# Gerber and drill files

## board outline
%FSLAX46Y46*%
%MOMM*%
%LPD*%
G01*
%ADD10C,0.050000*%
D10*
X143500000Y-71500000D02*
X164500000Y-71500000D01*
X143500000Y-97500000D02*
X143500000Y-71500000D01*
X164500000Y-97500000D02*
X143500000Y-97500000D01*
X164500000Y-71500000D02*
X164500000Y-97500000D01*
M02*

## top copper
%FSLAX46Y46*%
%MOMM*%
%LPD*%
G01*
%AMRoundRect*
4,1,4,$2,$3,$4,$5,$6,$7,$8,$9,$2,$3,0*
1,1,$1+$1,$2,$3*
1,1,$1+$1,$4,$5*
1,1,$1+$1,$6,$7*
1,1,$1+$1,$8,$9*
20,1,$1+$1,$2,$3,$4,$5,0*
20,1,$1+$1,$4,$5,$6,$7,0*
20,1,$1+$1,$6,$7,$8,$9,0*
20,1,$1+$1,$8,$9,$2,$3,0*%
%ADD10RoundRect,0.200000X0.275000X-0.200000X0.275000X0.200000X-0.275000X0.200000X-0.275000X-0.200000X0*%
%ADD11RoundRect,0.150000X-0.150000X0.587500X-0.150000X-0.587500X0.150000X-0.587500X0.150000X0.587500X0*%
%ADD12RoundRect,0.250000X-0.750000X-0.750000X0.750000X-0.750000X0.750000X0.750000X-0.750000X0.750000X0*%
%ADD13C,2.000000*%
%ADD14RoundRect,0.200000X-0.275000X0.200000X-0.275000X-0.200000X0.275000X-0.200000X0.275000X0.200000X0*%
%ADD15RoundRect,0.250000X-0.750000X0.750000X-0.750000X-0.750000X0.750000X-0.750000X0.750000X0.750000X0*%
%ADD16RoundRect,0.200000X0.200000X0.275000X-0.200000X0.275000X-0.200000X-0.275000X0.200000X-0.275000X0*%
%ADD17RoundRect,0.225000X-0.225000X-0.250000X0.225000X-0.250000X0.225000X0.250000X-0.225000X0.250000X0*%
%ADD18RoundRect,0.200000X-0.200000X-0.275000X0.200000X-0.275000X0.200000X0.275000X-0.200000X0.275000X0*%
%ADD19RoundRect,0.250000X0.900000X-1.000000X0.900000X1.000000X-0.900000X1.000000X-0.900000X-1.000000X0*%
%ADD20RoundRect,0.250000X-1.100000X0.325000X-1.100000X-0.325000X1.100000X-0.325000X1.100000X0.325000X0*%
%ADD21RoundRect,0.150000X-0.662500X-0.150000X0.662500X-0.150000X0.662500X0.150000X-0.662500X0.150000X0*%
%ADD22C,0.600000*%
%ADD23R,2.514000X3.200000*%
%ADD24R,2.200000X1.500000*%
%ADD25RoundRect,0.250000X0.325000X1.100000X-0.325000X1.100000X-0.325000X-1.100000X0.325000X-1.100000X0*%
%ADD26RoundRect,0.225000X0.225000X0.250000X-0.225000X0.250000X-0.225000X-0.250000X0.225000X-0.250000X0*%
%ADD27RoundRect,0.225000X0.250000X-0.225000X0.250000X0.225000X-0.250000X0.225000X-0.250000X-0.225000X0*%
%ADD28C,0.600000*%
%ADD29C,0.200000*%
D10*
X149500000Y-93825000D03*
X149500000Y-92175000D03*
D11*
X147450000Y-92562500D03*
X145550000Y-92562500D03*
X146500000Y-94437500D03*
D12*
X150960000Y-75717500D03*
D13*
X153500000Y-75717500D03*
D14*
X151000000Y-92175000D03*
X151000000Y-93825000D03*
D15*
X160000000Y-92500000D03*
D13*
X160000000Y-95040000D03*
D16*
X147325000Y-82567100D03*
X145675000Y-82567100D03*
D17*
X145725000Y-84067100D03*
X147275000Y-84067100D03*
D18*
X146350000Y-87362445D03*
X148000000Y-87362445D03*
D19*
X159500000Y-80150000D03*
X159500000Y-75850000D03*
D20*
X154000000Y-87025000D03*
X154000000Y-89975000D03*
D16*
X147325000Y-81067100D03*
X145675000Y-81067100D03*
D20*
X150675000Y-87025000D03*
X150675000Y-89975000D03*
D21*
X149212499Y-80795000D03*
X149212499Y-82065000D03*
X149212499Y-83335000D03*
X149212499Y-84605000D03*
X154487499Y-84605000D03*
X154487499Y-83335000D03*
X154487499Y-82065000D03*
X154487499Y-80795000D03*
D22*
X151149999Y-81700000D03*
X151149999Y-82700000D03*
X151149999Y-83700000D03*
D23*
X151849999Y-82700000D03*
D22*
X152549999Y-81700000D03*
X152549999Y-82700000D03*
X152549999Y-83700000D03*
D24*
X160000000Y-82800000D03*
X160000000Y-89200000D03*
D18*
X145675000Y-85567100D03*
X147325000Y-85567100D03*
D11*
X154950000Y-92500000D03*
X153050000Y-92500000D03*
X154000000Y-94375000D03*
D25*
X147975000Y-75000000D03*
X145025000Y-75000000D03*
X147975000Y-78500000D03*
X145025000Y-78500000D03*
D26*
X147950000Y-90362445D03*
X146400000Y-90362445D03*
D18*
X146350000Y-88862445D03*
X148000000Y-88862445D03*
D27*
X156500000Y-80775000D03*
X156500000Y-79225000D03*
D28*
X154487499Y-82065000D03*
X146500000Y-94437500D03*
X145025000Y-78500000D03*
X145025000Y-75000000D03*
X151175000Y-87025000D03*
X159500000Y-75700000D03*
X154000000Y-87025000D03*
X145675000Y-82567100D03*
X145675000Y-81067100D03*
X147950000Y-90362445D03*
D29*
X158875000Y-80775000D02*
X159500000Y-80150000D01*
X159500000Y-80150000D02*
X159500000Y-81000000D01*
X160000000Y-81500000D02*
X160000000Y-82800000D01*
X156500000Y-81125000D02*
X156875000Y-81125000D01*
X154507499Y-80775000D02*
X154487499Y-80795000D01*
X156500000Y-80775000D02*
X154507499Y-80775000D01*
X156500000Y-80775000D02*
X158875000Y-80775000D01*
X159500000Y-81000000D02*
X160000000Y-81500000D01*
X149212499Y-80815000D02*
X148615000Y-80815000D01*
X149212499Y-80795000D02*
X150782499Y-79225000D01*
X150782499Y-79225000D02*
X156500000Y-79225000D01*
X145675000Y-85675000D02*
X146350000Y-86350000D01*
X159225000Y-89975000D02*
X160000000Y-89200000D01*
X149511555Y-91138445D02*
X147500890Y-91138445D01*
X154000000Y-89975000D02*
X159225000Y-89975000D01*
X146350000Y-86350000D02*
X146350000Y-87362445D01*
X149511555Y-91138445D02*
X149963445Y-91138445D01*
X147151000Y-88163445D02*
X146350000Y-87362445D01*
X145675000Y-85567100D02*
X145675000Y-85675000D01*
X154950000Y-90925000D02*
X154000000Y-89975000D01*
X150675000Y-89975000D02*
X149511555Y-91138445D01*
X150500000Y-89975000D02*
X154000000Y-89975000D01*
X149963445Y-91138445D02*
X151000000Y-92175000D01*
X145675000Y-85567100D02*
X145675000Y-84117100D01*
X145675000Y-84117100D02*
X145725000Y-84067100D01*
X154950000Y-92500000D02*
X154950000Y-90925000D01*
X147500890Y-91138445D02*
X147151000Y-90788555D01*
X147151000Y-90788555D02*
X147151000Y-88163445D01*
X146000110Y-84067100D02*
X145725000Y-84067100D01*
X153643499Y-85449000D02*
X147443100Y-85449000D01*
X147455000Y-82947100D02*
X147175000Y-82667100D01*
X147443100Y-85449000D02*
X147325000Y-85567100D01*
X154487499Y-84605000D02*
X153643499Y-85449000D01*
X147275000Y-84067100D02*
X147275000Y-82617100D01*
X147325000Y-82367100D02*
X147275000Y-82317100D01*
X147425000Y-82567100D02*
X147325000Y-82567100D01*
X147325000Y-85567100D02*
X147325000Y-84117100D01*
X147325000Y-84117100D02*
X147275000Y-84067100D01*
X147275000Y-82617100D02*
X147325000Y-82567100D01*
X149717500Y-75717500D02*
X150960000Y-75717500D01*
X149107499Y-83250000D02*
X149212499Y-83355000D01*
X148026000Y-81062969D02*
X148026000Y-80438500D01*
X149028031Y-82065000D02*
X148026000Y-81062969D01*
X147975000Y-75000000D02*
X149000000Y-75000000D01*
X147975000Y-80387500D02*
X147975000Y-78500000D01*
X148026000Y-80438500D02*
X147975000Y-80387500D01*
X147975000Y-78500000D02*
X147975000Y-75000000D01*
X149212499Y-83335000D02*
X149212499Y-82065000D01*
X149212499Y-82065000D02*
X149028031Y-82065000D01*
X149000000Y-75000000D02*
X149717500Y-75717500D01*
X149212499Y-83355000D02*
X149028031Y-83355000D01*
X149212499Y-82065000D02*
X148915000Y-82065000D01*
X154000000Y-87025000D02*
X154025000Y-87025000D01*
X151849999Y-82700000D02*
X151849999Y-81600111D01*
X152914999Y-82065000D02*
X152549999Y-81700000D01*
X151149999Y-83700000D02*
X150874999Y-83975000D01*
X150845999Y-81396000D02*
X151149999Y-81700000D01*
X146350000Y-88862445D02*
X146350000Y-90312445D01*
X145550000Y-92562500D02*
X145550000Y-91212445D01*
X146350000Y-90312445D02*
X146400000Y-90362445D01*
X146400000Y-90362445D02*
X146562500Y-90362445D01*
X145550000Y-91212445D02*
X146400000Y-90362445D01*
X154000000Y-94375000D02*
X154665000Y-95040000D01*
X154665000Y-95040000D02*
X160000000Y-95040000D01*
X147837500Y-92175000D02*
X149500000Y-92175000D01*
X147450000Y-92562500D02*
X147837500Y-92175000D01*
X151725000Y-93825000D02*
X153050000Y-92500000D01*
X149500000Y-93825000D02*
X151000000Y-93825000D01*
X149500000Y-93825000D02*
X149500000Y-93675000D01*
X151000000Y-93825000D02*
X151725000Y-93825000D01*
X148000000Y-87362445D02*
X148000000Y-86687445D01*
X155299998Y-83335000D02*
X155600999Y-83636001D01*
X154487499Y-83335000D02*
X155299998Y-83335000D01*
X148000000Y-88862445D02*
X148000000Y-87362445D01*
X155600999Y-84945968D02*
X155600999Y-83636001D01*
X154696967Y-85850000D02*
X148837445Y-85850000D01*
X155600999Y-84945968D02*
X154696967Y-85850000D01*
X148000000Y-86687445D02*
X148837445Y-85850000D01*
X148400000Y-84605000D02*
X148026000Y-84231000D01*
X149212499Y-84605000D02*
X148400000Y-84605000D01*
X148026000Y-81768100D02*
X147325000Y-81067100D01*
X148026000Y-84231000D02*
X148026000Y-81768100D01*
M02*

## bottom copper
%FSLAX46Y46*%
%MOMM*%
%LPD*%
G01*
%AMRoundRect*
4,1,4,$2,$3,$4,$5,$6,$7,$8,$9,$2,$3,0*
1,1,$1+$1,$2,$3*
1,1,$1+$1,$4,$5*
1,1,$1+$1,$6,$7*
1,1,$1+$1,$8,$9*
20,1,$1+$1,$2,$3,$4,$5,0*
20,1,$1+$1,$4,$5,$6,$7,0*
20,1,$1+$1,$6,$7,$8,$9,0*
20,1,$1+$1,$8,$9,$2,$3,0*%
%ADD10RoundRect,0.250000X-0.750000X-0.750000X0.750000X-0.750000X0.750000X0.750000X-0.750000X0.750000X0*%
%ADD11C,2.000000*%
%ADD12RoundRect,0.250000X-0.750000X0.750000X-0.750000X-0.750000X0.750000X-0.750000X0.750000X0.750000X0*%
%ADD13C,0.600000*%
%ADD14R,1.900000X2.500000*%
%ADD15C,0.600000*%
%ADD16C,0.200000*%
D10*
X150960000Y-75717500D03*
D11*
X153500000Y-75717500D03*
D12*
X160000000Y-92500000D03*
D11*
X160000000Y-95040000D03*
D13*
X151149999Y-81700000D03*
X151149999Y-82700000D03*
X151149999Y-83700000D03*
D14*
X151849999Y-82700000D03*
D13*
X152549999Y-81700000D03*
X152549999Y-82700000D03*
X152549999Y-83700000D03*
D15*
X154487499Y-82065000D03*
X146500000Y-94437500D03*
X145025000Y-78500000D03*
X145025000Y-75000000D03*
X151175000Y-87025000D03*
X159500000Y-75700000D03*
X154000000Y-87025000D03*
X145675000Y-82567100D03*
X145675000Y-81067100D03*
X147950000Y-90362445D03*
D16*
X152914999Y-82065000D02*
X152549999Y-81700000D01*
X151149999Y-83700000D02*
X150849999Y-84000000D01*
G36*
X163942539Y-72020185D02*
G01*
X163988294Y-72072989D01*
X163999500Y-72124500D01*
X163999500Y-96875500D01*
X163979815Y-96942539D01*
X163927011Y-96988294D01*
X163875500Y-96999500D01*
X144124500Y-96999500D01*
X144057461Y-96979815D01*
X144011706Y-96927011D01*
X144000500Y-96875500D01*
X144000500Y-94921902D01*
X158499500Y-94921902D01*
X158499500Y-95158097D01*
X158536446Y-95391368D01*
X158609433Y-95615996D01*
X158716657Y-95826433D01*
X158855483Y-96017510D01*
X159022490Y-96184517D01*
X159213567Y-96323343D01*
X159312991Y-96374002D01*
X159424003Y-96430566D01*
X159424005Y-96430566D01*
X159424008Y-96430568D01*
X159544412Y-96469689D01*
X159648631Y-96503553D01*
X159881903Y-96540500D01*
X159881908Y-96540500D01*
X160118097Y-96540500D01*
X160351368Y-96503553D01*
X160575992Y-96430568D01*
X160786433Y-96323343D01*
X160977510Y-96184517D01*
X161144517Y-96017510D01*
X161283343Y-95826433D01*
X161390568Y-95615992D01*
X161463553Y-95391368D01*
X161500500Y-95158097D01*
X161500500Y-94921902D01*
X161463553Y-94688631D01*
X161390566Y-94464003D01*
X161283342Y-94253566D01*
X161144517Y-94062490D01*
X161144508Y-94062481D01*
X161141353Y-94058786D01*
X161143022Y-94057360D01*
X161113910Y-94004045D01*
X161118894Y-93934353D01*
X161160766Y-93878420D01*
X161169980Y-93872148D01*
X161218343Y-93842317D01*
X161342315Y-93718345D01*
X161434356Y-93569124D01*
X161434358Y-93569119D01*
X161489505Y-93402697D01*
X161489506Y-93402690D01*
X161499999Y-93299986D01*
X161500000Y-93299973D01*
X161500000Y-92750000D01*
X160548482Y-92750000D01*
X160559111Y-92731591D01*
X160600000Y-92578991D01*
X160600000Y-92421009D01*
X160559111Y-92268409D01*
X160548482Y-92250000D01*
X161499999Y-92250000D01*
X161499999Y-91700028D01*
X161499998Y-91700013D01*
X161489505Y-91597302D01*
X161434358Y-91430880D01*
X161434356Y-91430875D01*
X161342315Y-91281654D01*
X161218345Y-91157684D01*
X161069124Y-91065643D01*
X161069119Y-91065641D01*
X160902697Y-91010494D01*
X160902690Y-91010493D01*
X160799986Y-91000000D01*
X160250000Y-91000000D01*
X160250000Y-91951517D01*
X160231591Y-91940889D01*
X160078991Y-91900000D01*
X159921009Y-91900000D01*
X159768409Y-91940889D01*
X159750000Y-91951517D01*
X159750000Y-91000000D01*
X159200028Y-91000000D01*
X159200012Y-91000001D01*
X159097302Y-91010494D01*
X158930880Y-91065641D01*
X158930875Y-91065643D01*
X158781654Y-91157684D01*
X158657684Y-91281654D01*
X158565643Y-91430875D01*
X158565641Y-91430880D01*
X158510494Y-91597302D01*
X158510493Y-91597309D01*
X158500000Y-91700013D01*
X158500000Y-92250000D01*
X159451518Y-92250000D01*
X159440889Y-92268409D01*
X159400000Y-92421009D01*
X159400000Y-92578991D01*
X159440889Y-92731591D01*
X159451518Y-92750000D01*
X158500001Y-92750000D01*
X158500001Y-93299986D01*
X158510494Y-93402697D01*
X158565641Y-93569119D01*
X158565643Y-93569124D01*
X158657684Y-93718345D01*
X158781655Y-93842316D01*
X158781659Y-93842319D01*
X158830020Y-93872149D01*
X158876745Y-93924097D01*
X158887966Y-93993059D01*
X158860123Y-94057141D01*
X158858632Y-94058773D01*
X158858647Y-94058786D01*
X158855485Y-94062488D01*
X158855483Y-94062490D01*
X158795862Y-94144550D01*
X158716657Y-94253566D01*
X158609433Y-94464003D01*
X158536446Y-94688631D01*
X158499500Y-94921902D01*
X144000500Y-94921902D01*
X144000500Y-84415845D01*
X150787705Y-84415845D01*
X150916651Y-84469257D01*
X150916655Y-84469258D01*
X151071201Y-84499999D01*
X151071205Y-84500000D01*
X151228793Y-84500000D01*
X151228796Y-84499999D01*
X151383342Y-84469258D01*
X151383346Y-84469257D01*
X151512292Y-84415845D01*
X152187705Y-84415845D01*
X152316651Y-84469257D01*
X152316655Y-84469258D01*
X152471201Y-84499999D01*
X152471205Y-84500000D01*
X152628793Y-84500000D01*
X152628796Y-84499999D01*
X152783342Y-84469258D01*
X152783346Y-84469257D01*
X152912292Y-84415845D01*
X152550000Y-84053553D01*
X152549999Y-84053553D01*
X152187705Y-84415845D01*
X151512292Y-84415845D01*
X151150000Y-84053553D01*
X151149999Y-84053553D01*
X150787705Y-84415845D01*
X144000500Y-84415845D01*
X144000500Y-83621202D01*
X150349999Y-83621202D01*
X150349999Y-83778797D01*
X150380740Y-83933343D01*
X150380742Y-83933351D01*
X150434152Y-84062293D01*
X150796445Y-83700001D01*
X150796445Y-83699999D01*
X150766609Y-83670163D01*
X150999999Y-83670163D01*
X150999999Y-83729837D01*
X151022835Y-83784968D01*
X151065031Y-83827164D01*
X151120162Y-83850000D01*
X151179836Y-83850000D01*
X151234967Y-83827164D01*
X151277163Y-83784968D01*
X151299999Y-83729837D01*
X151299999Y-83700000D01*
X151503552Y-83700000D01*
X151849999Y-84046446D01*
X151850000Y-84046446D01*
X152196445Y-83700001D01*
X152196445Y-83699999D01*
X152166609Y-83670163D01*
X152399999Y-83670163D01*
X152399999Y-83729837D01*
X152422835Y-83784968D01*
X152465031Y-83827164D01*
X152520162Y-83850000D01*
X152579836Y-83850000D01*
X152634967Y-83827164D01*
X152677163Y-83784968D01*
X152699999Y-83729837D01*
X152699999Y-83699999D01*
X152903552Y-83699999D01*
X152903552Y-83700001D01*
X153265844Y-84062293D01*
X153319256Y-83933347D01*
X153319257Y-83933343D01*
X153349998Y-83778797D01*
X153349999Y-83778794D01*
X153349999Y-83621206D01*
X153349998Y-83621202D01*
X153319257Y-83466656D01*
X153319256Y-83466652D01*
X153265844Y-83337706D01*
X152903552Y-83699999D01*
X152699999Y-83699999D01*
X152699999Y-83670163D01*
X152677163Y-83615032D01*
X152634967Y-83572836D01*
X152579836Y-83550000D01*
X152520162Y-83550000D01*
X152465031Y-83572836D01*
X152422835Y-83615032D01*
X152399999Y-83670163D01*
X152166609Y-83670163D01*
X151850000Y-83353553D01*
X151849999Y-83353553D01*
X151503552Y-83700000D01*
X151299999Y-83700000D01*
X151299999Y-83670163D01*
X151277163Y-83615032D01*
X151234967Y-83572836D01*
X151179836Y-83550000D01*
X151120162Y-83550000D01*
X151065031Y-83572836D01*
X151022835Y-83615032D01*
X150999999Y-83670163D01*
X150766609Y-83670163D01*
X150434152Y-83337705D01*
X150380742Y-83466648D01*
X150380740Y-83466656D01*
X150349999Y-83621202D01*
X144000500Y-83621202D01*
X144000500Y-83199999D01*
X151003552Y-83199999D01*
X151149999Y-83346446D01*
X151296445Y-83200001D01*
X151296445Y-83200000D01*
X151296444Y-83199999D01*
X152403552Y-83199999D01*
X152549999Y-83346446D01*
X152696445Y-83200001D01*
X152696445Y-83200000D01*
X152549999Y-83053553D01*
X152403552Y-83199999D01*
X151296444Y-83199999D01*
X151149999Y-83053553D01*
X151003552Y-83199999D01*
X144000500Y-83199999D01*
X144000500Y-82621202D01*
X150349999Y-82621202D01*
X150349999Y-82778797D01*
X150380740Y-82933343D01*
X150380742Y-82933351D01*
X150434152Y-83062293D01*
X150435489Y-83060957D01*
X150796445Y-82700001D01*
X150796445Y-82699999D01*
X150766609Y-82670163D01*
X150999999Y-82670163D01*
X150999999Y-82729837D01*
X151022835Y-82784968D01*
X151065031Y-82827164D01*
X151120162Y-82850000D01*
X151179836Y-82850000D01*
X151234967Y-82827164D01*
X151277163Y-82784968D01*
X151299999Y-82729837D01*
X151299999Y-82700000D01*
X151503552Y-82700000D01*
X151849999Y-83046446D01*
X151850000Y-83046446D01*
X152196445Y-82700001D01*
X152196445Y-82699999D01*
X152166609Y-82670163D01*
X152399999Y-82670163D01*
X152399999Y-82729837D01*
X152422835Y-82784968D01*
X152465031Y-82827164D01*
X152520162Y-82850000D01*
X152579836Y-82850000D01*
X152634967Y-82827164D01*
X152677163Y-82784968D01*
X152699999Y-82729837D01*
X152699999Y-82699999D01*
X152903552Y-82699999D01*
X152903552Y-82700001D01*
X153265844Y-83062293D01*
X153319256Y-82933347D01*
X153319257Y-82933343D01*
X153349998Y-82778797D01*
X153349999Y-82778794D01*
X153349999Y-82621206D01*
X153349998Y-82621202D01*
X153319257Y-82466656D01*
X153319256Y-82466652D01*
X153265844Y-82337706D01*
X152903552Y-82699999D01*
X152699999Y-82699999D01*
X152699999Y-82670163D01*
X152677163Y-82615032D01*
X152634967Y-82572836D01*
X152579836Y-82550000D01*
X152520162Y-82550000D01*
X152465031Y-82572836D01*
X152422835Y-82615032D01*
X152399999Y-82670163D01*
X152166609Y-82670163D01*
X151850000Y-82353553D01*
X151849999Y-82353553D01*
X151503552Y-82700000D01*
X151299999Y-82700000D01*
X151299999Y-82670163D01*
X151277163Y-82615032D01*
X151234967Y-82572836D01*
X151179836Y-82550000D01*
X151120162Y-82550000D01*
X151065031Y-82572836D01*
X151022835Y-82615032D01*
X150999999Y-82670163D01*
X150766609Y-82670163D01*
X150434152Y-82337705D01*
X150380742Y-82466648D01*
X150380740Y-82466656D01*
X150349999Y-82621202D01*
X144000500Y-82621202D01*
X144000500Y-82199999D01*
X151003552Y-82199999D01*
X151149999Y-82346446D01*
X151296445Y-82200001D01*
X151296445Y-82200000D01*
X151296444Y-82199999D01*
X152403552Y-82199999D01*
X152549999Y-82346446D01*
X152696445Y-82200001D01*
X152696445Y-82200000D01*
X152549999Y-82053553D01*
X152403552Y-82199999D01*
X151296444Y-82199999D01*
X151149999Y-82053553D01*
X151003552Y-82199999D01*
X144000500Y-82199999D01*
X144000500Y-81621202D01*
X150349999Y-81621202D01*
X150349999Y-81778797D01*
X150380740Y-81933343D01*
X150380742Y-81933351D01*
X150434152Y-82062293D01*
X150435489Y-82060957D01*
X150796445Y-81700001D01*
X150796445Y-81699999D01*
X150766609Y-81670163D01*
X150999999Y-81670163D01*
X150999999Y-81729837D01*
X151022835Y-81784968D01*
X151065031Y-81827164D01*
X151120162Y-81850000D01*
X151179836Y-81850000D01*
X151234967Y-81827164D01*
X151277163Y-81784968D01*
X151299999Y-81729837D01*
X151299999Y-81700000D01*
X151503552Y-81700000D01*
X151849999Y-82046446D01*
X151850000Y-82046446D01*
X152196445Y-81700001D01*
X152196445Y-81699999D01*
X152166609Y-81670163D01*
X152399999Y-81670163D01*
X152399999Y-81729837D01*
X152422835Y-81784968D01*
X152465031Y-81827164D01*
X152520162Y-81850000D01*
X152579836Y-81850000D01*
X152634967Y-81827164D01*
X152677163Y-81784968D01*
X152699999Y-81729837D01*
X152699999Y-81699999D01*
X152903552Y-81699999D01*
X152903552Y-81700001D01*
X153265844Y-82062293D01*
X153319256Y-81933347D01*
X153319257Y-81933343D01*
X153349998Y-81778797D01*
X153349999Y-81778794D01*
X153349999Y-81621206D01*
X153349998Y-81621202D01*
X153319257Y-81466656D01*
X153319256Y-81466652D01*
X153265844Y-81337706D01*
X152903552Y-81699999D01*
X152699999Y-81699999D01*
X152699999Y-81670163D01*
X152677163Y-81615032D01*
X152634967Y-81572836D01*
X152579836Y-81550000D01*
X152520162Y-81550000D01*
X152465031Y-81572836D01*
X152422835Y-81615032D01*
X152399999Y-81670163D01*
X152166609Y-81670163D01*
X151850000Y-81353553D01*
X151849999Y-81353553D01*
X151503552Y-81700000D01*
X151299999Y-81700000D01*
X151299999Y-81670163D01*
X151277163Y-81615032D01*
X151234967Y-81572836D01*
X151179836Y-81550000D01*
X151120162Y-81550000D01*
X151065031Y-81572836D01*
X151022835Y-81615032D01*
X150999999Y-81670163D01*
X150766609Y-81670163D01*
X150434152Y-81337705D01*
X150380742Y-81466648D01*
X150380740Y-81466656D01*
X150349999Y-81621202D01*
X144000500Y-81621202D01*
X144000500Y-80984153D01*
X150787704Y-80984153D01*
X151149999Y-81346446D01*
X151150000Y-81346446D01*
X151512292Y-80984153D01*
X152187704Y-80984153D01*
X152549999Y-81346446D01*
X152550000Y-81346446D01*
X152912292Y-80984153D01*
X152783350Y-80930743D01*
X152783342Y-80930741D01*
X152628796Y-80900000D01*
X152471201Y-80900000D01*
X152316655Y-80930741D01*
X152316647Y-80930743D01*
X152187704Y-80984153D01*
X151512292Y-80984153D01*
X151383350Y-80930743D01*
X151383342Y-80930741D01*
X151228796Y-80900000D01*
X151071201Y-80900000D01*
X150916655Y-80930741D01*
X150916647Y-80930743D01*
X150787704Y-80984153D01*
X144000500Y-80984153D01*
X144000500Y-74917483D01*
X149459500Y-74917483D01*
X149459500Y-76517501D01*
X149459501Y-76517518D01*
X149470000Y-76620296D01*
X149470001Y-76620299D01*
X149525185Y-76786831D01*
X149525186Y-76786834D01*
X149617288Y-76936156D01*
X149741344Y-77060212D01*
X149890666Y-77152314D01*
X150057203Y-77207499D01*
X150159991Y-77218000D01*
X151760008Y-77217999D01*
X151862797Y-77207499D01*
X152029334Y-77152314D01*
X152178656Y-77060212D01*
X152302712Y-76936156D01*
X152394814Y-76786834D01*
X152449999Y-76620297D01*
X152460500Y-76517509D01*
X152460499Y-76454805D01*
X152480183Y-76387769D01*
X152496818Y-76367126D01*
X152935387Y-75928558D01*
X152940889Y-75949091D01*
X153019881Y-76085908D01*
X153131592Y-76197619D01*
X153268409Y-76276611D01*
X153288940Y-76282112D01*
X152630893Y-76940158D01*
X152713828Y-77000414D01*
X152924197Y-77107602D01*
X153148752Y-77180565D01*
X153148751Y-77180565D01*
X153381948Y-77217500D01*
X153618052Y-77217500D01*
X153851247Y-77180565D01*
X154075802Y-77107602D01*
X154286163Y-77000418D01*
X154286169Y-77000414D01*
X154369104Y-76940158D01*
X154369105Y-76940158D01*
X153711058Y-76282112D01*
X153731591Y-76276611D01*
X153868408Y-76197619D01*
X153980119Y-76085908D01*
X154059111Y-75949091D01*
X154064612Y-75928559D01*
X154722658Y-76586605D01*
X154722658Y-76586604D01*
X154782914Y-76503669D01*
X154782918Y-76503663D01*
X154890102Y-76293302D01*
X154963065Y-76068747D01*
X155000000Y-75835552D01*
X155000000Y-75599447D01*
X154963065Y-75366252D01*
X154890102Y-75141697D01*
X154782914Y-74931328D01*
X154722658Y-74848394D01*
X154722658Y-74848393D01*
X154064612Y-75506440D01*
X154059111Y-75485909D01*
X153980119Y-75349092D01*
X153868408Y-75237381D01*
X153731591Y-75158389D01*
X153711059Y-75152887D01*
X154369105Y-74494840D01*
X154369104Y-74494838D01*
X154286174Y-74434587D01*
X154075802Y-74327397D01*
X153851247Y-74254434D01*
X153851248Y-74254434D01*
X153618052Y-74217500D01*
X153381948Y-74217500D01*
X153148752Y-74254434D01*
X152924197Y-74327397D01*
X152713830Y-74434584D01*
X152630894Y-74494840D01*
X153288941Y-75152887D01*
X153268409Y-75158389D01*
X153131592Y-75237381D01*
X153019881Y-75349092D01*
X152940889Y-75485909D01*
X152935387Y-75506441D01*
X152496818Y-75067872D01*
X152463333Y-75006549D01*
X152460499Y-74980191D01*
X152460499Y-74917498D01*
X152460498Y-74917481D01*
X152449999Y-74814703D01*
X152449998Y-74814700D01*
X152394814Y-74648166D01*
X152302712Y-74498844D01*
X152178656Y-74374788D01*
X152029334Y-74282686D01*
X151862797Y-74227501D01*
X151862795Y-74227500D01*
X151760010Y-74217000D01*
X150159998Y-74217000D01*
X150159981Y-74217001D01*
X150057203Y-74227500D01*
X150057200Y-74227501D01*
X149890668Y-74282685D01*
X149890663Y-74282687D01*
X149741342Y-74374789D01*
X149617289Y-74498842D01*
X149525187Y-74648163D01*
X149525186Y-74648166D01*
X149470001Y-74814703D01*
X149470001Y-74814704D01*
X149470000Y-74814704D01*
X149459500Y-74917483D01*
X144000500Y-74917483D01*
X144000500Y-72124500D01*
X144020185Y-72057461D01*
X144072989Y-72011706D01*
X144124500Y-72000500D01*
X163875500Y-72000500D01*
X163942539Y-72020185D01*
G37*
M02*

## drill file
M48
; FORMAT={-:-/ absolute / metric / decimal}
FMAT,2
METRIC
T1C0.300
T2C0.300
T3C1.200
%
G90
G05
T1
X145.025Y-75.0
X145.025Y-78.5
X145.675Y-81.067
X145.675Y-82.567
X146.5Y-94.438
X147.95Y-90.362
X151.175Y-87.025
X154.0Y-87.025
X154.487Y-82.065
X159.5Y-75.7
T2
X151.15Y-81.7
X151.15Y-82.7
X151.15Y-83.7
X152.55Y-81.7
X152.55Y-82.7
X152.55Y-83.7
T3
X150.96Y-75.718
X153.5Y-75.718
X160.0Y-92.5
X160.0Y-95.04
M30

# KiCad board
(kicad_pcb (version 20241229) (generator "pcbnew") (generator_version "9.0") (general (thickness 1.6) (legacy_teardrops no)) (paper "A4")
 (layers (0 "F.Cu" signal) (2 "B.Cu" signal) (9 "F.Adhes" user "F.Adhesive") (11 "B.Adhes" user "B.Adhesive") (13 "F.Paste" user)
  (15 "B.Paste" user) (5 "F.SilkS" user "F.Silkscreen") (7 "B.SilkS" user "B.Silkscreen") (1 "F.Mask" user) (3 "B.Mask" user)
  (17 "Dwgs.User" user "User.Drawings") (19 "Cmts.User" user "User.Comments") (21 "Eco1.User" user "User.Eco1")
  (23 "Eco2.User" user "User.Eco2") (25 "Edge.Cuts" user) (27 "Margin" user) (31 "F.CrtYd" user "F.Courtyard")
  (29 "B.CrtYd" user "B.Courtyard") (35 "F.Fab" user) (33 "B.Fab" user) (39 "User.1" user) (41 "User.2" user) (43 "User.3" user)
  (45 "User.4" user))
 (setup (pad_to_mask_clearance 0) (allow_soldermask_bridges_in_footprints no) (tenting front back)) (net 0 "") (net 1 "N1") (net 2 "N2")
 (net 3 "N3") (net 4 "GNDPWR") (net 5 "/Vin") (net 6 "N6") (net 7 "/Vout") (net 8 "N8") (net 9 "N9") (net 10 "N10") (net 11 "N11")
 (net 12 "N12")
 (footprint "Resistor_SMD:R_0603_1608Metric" (layer "F.Cu") (at 149.5 93 90)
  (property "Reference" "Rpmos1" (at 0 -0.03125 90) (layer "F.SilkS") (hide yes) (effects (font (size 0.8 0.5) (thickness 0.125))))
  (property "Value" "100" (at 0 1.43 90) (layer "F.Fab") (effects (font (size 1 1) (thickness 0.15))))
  (pad "1" smd roundrect (at -0.825 0 90) (size 0.8 0.95) (layers "F.Cu" "F.Mask" "F.Paste") (roundrect_rratio 0.25) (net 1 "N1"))
  (pad "2" smd roundrect (at 0.825 0 90) (size 0.8 0.95) (layers "F.Cu" "F.Mask" "F.Paste") (roundrect_rratio 0.25) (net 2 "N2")))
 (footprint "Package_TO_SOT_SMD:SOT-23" (layer "F.Cu") (at 146.5 93.5 -90)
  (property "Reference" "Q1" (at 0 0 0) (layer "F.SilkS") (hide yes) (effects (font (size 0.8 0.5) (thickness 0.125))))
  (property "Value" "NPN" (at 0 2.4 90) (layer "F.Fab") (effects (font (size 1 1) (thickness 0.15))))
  (pad "1" smd roundrect (at -0.9375 -0.95 270) (size 1.475 0.6) (layers "F.Cu" "F.Mask" "F.Paste") (roundrect_rratio 0.25) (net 2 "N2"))
  (pad "2" smd roundrect (at -0.9375 0.95 270) (size 1.475 0.6) (layers "F.Cu" "F.Mask" "F.Paste") (roundrect_rratio 0.25) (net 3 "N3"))
  (pad "3" smd roundrect (at 0.9375 0 270) (size 1.475 0.6) (layers "F.Cu" "F.Mask" "F.Paste") (roundrect_rratio 0.25) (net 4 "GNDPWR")))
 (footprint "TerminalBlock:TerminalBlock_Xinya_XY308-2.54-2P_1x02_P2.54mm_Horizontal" (layer "F.Cu") (at 150.96 75.7175)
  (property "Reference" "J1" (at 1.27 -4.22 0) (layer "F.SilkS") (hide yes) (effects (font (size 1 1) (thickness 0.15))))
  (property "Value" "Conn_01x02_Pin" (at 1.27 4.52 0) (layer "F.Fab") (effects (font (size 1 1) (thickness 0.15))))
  (pad "1" thru_hole roundrect (at 0 0) (size 2 2) (drill 1.2) (layers "*.Cu" "*.Mask") (remove_unused_layers no) (roundrect_rratio 0.125)
   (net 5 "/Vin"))
  (pad "2" thru_hole circle (at 2.54 0) (size 2 2) (drill 1.2) (layers "*.Cu" "*.Mask") (remove_unused_layers no) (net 4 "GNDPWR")))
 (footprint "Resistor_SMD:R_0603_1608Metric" (layer "F.Cu") (at 151 93 -90)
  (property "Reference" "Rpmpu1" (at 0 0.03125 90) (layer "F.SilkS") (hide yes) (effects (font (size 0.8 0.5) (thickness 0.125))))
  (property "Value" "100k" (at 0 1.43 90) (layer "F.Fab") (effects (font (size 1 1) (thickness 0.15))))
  (pad "1" smd roundrect (at -0.825 0 270) (size 0.8 0.95) (layers "F.Cu" "F.Mask" "F.Paste") (roundrect_rratio 0.25) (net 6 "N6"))
  (pad "2" smd roundrect (at 0.825 0 270) (size 0.8 0.95) (layers "F.Cu" "F.Mask" "F.Paste") (roundrect_rratio 0.25) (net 1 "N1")))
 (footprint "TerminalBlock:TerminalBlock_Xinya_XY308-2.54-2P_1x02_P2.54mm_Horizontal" (layer "F.Cu") (at 160 92.5 -90)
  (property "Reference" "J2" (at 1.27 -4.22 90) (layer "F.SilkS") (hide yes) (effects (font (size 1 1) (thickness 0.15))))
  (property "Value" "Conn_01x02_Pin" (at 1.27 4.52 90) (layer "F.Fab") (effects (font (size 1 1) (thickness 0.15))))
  (pad "1" thru_hole roundrect (at 0 0 270) (size 2 2) (drill 1.2) (layers "*.Cu" "*.Mask") (remove_unused_layers no)
   (roundrect_rratio 0.125) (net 4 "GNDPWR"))
  (pad "2" thru_hole circle (at 2.54 0 270) (size 2 2) (drill 1.2) (layers "*.Cu" "*.Mask") (remove_unused_layers no) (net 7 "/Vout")))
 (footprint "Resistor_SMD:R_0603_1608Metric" (layer "F.Cu") (at 146.5 82.5671 180)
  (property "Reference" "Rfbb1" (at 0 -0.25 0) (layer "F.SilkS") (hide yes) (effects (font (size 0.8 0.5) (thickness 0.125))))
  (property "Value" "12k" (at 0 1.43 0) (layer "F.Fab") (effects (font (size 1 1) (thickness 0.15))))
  (pad "1" smd roundrect (at -0.825 0 180) (size 0.8 0.95) (layers "F.Cu" "F.Mask" "F.Paste") (roundrect_rratio 0.25) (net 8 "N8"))
  (pad "2" smd roundrect (at 0.825 0 180) (size 0.8 0.95) (layers "F.Cu" "F.Mask" "F.Paste") (roundrect_rratio 0.25) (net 4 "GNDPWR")))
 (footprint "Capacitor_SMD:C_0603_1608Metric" (layer "F.Cu") (at 146.5 84.0671)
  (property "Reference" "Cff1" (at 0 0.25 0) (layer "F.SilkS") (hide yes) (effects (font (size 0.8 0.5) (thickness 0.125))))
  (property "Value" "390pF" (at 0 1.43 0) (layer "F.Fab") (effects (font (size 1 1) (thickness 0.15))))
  (pad "1" smd roundrect (at -0.775 0) (size 0.9 0.95) (layers "F.Cu" "F.Mask" "F.Paste") (roundrect_rratio 0.25) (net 6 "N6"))
  (pad "2" smd roundrect (at 0.775 0) (size 0.9 0.95) (layers "F.Cu" "F.Mask" "F.Paste") (roundrect_rratio 0.25) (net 8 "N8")))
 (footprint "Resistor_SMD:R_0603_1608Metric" (layer "F.Cu") (at 147.175 87.362445)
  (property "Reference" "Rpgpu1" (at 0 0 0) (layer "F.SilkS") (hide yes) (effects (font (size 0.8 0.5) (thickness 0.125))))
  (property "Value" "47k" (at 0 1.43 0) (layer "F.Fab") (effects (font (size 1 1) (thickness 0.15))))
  (pad "1" smd roundrect (at -0.825 0) (size 0.8 0.95) (layers "F.Cu" "F.Mask" "F.Paste") (roundrect_rratio 0.25) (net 6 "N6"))
  (pad "2" smd roundrect (at 0.825 0) (size 0.8 0.95) (layers "F.Cu" "F.Mask" "F.Paste") (roundrect_rratio 0.25) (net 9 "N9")))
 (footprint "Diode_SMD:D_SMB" (layer "F.Cu") (at 159.5 78 90)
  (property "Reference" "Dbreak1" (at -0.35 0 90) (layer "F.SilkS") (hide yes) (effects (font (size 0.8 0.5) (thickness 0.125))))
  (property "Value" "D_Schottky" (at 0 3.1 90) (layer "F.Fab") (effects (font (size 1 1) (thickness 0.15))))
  (pad "1" smd roundrect (at -2.15 0 90) (size 2.5 2.3) (layers "F.Cu" "F.Mask" "F.Paste") (roundrect_rratio 0.1086956522) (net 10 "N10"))
  (pad "2" smd roundrect (at 2.15 0 90) (size 2.5 2.3) (layers "F.Cu" "F.Mask" "F.Paste") (roundrect_rratio 0.1086956522) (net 4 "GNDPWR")))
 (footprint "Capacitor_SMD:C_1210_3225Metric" (layer "F.Cu") (at 154 88.5 -90)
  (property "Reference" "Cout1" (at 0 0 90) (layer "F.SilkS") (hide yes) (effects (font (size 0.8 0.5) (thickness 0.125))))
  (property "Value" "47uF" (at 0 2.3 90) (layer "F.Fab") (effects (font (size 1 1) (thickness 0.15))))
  (pad "1" smd roundrect (at -1.475 0 270) (size 1.15 2.7) (layers "F.Cu" "F.Mask" "F.Paste") (roundrect_rratio 0.217391) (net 4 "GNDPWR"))
  (pad "2" smd roundrect (at 1.475 0 270) (size 1.15 2.7) (layers "F.Cu" "F.Mask" "F.Paste") (roundrect_rratio 0.217391) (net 6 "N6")))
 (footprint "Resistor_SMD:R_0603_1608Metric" (layer "F.Cu") (at 146.5 81.0671 180)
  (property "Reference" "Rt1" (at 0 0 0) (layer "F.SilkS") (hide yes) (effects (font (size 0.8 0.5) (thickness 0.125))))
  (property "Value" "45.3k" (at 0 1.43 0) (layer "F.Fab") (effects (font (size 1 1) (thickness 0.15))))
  (pad "1" smd roundrect (at -0.825 0 180) (size 0.8 0.95) (layers "F.Cu" "F.Mask" "F.Paste") (roundrect_rratio 0.25) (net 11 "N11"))
  (pad "2" smd roundrect (at 0.825 0 180) (size 0.8 0.95) (layers "F.Cu" "F.Mask" "F.Paste") (roundrect_rratio 0.25) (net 4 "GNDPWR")))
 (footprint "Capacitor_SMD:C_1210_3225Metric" (layer "F.Cu") (at 150.675 88.5 -90)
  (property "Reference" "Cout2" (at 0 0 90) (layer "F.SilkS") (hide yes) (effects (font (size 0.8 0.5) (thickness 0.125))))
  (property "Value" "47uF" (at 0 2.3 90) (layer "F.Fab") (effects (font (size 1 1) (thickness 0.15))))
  (pad "1" smd roundrect (at -1.475 0 270) (size 1.15 2.7) (layers "F.Cu" "F.Mask" "F.Paste") (roundrect_rratio 0.217391) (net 4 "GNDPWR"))
  (pad "2" smd roundrect (at 1.475 0 270) (size 1.15 2.7) (layers "F.Cu" "F.Mask" "F.Paste") (roundrect_rratio 0.217391) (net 6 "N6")))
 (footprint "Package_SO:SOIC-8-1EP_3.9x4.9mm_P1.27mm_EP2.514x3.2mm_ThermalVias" (layer "F.Cu") (at 151.849999 82.7)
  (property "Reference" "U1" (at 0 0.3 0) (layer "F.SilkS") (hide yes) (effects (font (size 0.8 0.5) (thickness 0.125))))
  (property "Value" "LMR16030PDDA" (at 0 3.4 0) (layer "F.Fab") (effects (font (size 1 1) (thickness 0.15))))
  (pad "" smd roundrect (at -0.63 -0.8) (size 1.05 1.34) (layers "F.Paste") (roundrect_rratio 0.238095))
  (pad "" smd roundrect (at -0.63 0.8) (size 1.05 1.34) (layers "F.Paste") (roundrect_rratio 0.238095))
  (pad "" smd roundrect (at 0.63 -0.8) (size 1.05 1.34) (layers "F.Paste") (roundrect_rratio 0.238095))
  (pad "" smd roundrect (at 0.63 0.8) (size 1.05 1.34) (layers "F.Paste") (roundrect_rratio 0.238095))
  (pad "1" smd roundrect (at -2.6375 -1.905) (size 1.625 0.6) (layers "F.Cu" "F.Mask" "F.Paste") (roundrect_rratio 0.25) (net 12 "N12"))
  (pad "2" smd roundrect (at -2.6375 -0.635) (size 1.625 0.6) (layers "F.Cu" "F.Mask" "F.Paste") (roundrect_rratio 0.25) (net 5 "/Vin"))
  (pad "3" smd roundrect (at -2.6375 0.635) (size 1.625 0.6) (layers "F.Cu" "F.Mask" "F.Paste") (roundrect_rratio 0.25) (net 5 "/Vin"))
  (pad "4" smd roundrect (at -2.6375 1.905) (size 1.625 0.6) (layers "F.Cu" "F.Mask" "F.Paste") (roundrect_rratio 0.25) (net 11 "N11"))
  (pad "5" smd roundrect (at 2.6375 1.905) (size 1.625 0.6) (layers "F.Cu" "F.Mask" "F.Paste") (roundrect_rratio 0.25) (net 8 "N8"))
  (pad "6" smd roundrect (at 2.6375 0.635) (size 1.625 0.6) (layers "F.Cu" "F.Mask" "F.Paste") (roundrect_rratio 0.25) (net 9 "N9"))
  (pad "7" smd roundrect (at 2.6375 -0.635) (size 1.625 0.6) (layers "F.Cu" "F.Mask" "F.Paste") (roundrect_rratio 0.25) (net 4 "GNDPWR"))
  (pad "8" smd roundrect (at 2.6375 -1.905) (size 1.625 0.6) (layers "F.Cu" "F.Mask" "F.Paste") (roundrect_rratio 0.25) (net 10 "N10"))
  (pad "9" thru_hole circle (at -0.7 -1) (size 0.6 0.6) (drill 0.3) (layers "*.Cu") (remove_unused_layers no) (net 4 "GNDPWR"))
  (pad "9" thru_hole circle (at -0.7 0) (size 0.6 0.6) (drill 0.3) (layers "*.Cu") (remove_unused_layers no) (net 4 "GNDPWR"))
  (pad "9" thru_hole circle (at -0.7 1) (size 0.6 0.6) (drill 0.3) (layers "*.Cu") (remove_unused_layers no) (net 4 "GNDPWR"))
  (pad "9" smd rect (at 0 0) (size 1.9 2.5) (layers "B.Cu") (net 4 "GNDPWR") (zone_connect 2))
  (pad "9" smd rect (at 0 0) (size 2.514 3.2) (layers "F.Cu" "F.Mask") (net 4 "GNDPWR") (zone_connect 2))
  (pad "9" thru_hole circle (at 0.7 -1) (size 0.6 0.6) (drill 0.3) (layers "*.Cu") (remove_unused_layers no) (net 4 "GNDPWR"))
  (pad "9" thru_hole circle (at 0.7 0) (size 0.6 0.6) (drill 0.3) (layers "*.Cu") (remove_unused_layers no) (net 4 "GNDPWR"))
  (pad "9" thru_hole circle (at 0.7 1) (size 0.6 0.6) (drill 0.3) (layers "*.Cu") (remove_unused_layers no) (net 4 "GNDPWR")))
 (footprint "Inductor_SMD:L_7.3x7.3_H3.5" (layer "F.Cu") (at 160 86 -90)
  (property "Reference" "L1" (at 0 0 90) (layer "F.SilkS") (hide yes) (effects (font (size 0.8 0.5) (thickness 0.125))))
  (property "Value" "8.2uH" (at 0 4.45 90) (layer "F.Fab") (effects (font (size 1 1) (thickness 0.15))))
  (pad "1" smd rect (at -3.2 0 270) (size 1.5 2.2) (layers "F.Cu" "F.Mask" "F.Paste") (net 10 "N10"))
  (pad "2" smd rect (at 3.2 0 270) (size 1.5 2.2) (layers "F.Cu" "F.Mask" "F.Paste") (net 6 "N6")))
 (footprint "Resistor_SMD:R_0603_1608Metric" (layer "F.Cu") (at 146.5 85.5671)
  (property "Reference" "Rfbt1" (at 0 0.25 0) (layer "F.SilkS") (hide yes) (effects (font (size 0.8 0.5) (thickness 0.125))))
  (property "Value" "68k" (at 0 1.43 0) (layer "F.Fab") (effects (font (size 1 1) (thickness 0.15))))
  (pad "1" smd roundrect (at -0.825 0) (size 0.8 0.95) (layers "F.Cu" "F.Mask" "F.Paste") (roundrect_rratio 0.25) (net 6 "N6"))
  (pad "2" smd roundrect (at 0.825 0) (size 0.8 0.95) (layers "F.Cu" "F.Mask" "F.Paste") (roundrect_rratio 0.25) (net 8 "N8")))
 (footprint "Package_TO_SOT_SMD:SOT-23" (layer "F.Cu") (at 154 93.4375 -90)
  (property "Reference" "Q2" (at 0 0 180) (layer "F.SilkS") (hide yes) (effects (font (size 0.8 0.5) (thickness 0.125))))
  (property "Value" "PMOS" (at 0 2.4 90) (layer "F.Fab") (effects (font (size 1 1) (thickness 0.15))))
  (pad "1" smd roundrect (at -0.9375 -0.95 270) (size 1.475 0.6) (layers "F.Cu" "F.Mask" "F.Paste") (roundrect_rratio 0.25) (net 6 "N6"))
  (pad "2" smd roundrect (at -0.9375 0.95 270) (size 1.475 0.6) (layers "F.Cu" "F.Mask" "F.Paste") (roundrect_rratio 0.25) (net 1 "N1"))
  (pad "3" smd roundrect (at 0.9375 0 270) (size 1.475 0.6) (layers "F.Cu" "F.Mask" "F.Paste") (roundrect_rratio 0.25) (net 7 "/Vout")))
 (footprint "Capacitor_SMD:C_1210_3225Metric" (layer "F.Cu") (at 146.5 75 180)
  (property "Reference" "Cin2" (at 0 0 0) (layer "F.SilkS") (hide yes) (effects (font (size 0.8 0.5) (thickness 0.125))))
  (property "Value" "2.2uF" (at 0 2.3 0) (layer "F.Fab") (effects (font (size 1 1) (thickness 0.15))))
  (pad "1" smd roundrect (at -1.475 0 180) (size 1.15 2.7) (layers "F.Cu" "F.Mask" "F.Paste") (roundrect_rratio 0.217391) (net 5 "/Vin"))
  (pad "2" smd roundrect (at 1.475 0 180) (size 1.15 2.7) (layers "F.Cu" "F.Mask" "F.Paste") (roundrect_rratio 0.217391) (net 4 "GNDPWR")))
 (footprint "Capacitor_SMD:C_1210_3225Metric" (layer "F.Cu") (at 146.5 78.5 180)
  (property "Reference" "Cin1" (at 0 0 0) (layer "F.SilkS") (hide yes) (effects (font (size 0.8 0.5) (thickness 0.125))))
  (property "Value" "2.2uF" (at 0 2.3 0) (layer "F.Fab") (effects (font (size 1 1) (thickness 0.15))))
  (pad "1" smd roundrect (at -1.475 0 180) (size 1.15 2.7) (layers "F.Cu" "F.Mask" "F.Paste") (roundrect_rratio 0.217391) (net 5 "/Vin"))
  (pad "2" smd roundrect (at 1.475 0 180) (size 1.15 2.7) (layers "F.Cu" "F.Mask" "F.Paste") (roundrect_rratio 0.217391) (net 4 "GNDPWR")))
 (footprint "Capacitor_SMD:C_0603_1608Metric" (layer "F.Cu") (at 147.175 90.362445 180)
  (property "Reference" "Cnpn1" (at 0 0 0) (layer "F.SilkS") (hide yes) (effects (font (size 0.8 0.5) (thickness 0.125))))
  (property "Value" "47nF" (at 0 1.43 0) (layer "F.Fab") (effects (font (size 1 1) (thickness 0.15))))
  (pad "1" smd roundrect (at -0.775 0 180) (size 0.9 0.95) (layers "F.Cu" "F.Mask" "F.Paste") (roundrect_rratio 0.25) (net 4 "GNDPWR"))
  (pad "2" smd roundrect (at 0.775 0 180) (size 0.9 0.95) (layers "F.Cu" "F.Mask" "F.Paste") (roundrect_rratio 0.25) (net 3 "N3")))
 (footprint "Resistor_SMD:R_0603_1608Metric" (layer "F.Cu") (at 147.175 88.862445)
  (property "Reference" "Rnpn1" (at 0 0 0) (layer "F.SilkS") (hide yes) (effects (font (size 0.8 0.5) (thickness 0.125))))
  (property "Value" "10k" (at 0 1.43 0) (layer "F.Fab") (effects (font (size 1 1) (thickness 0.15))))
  (pad "1" smd roundrect (at -0.825 0) (size 0.8 0.95) (layers "F.Cu" "F.Mask" "F.Paste") (roundrect_rratio 0.25) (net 3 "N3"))
  (pad "2" smd roundrect (at 0.825 0) (size 0.8 0.95) (layers "F.Cu" "F.Mask" "F.Paste") (roundrect_rratio 0.25) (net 9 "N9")))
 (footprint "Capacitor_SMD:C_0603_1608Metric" (layer "F.Cu") (at 156.5 80 90)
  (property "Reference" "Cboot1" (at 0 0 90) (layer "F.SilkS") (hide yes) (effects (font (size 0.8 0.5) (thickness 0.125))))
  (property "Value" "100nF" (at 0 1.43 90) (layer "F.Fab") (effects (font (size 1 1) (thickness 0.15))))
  (pad "1" smd roundrect (at -0.775 0 90) (size 0.9 0.95) (layers "F.Cu" "F.Mask" "F.Paste") (roundrect_rratio 0.25) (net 10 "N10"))
  (pad "2" smd roundrect (at 0.775 0 90) (size 0.9 0.95) (layers "F.Cu" "F.Mask" "F.Paste") (roundrect_rratio 0.25) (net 12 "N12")))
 (gr_line (start 143.5 71.5) (end 164.5 71.5) (stroke (width 0.05) (type default)) (layer "Edge.Cuts"))
 (gr_line (start 143.5 97.5) (end 143.5 71.5) (stroke (width 0.05) (type default)) (layer "Edge.Cuts"))
 (gr_line (start 164.5 97.5) (end 143.5 97.5) (stroke (width 0.05) (type default)) (layer "Edge.Cuts"))
 (gr_line (start 164.5 71.5) (end 164.5 97.5) (stroke (width 0.05) (type default)) (layer "Edge.Cuts"))
 (segment (start 158.875 80.775) (end 159.5 80.15) (width 0.2) (layer "F.Cu") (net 10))
 (segment (start 159.5 80.15) (end 159.5 81) (width 0.2) (layer "F.Cu") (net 10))
 (segment (start 160 81.5) (end 160 82.8) (width 0.2) (layer "F.Cu") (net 10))
 (segment (start 156.5 81.125) (end 156.875 81.125) (width 0.2) (layer "F.Cu") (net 10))
 (segment (start 154.507499 80.775) (end 154.487499 80.795) (width 0.2) (layer "F.Cu") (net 10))
 (segment (start 156.5 80.775) (end 154.507499 80.775) (width 0.2) (layer "F.Cu") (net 10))
 (segment (start 156.5 80.775) (end 158.875 80.775) (width 0.2) (layer "F.Cu") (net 10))
 (segment (start 159.5 81) (end 160 81.5) (width 0.2) (layer "F.Cu") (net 10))
 (segment (start 149.212499 80.815) (end 148.615 80.815) (width 0.2) (layer "F.Cu") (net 12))
 (segment (start 149.212499 80.795) (end 150.782499 79.225) (width 0.2) (layer "F.Cu") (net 12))
 (segment (start 150.782499 79.225) (end 156.5 79.225) (width 0.2) (layer "F.Cu") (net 12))
 (segment (start 145.675 85.675) (end 146.35 86.35) (width 0.2) (layer "F.Cu") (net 6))
 (segment (start 159.225 89.975) (end 160 89.2) (width 0.2) (layer "F.Cu") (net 6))
 (segment (start 149.511555 91.138445) (end 147.50089 91.138445) (width 0.2) (layer "F.Cu") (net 6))
 (segment (start 154 89.975) (end 159.225 89.975) (width 0.2) (layer "F.Cu") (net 6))
 (segment (start 146.35 86.35) (end 146.35 87.362445) (width 0.2) (layer "F.Cu") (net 6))
 (segment (start 149.511555 91.138445) (end 149.963445 91.138445) (width 0.2) (layer "F.Cu") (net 6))
 (segment (start 147.151 88.163445) (end 146.35 87.362445) (width 0.2) (layer "F.Cu") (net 6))
 (segment (start 145.675 85.5671) (end 145.675 85.675) (width 0.2) (layer "F.Cu") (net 6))
 (segment (start 154.95 90.925) (end 154 89.975) (width 0.2) (layer "F.Cu") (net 6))
 (segment (start 150.675 89.975) (end 149.511555 91.138445) (width 0.2) (layer "F.Cu") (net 6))
 (segment (start 150.5 89.975) (end 154 89.975) (width 0.2) (layer "F.Cu") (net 6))
 (segment (start 149.963445 91.138445) (end 151 92.175) (width 0.2) (layer "F.Cu") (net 6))
 (segment (start 145.675 85.5671) (end 145.675 84.1171) (width 0.2) (layer "F.Cu") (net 6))
 (segment (start 145.675 84.1171) (end 145.725 84.0671) (width 0.2) (layer "F.Cu") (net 6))
 (segment (start 154.95 92.5) (end 154.95 90.925) (width 0.2) (layer "F.Cu") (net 6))
 (segment (start 147.50089 91.138445) (end 147.151 90.788555) (width 0.2) (layer "F.Cu") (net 6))
 (segment (start 147.151 90.788555) (end 147.151 88.163445) (width 0.2) (layer "F.Cu") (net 6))
 (segment (start 146.00011 84.0671) (end 145.725 84.0671) (width 0.2) (layer "F.Cu") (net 6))
 (segment (start 153.643499 85.449) (end 147.4431 85.449) (width 0.2) (layer "F.Cu") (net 8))
 (segment (start 147.455 82.9471) (end 147.175 82.6671) (width 0.2) (layer "F.Cu") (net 8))
 (segment (start 147.4431 85.449) (end 147.325 85.5671) (width 0.2) (layer "F.Cu") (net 8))
 (segment (start 154.487499 84.605) (end 153.643499 85.449) (width 0.2) (layer "F.Cu") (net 8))
 (segment (start 147.275 84.0671) (end 147.275 82.6171) (width 0.2) (layer "F.Cu") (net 8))
 (segment (start 147.325 82.3671) (end 147.275 82.3171) (width 0.2) (layer "F.Cu") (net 8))
 (segment (start 147.425 82.5671) (end 147.325 82.5671) (width 0.2) (layer "F.Cu") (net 8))
 (segment (start 147.325 85.5671) (end 147.325 84.1171) (width 0.2) (layer "F.Cu") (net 8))
 (segment (start 147.325 84.1171) (end 147.275 84.0671) (width 0.2) (layer "F.Cu") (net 8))
 (segment (start 147.275 82.6171) (end 147.325 82.5671) (width 0.2) (layer "F.Cu") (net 8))
 (segment (start 149.7175 75.7175) (end 150.96 75.7175) (width 0.2) (layer "F.Cu") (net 5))
 (segment (start 149.107499 83.25) (end 149.212499 83.355) (width 0.2) (layer "F.Cu") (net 5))
 (segment (start 148.026 81.062969) (end 148.026 80.4385) (width 0.2) (layer "F.Cu") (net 5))
 (segment (start 149.028031 82.065) (end 148.026 81.062969) (width 0.2) (layer "F.Cu") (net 5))
 (segment (start 147.975 75) (end 149 75) (width 0.2) (layer "F.Cu") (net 5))
 (segment (start 147.975 80.3875) (end 147.975 78.5) (width 0.2) (layer "F.Cu") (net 5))
 (segment (start 148.026 80.4385) (end 147.975 80.3875) (width 0.2) (layer "F.Cu") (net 5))
 (segment (start 147.975 78.5) (end 147.975 75) (width 0.2) (layer "F.Cu") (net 5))
 (segment (start 149.212499 83.335) (end 149.212499 82.065) (width 0.2) (layer "F.Cu") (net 5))
 (segment (start 149.212499 82.065) (end 149.028031 82.065) (width 0.2) (layer "F.Cu") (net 5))
 (segment (start 149 75) (end 149.7175 75.7175) (width 0.2) (layer "F.Cu") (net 5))
 (segment (start 149.212499 83.355) (end 149.028031 83.355) (width 0.2) (layer "F.Cu") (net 5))
 (segment (start 149.212499 82.065) (end 148.915 82.065) (width 0.2) (layer "F.Cu") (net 5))
 (segment (start 154 87.025) (end 154.025 87.025) (width 0.2) (layer "F.Cu") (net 4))
 (segment (start 151.849999 82.7) (end 151.849999 81.600111) (width 0.2) (layer "F.Cu") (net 4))
 (segment (start 152.914999 82.065) (end 152.549999 81.7) (width 0.2) (layer "F.Cu") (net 4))
 (segment (start 151.149999 83.7) (end 150.874999 83.975) (width 0.2) (layer "F.Cu") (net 4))
 (segment (start 150.845999 81.396) (end 151.149999 81.7) (width 0.2) (layer "F.Cu") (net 4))
 (via (at 154.487499 82.065) (size 0.6) (drill 0.3) (layers "F.Cu" "B.Cu") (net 4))
 (via (at 146.5 94.4375) (size 0.6) (drill 0.3) (layers "F.Cu" "B.Cu") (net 4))
 (via (at 145.025 78.5) (size 0.6) (drill 0.3) (layers "F.Cu" "B.Cu") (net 4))
 (via (at 145.025 75) (size 0.6) (drill 0.3) (layers "F.Cu" "B.Cu") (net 4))
 (via (at 151.175 87.025) (size 0.6) (drill 0.3) (layers "F.Cu" "B.Cu") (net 4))
 (via (at 159.5 75.7) (size 0.6) (drill 0.3) (layers "F.Cu" "B.Cu") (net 4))
 (via (at 154 87.025) (size 0.6) (drill 0.3) (layers "F.Cu" "B.Cu") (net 4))
 (via (at 145.675 82.5671) (size 0.6) (drill 0.3) (layers "F.Cu" "B.Cu") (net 4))
 (via (at 145.675 81.0671) (size 0.6) (drill 0.3) (layers "F.Cu" "B.Cu") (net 4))
 (via (at 147.95 90.362445) (size 0.6) (drill 0.3) (layers "F.Cu" "B.Cu") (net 4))
 (segment (start 152.914999 82.065) (end 152.549999 81.7) (width 0.2) (layer "B.Cu") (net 4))
 (segment (start 151.149999 83.7) (end 150.849999 84) (width 0.2) (layer "B.Cu") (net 4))
 (segment (start 146.35 88.862445) (end 146.35 90.312445) (width 0.2) (layer "F.Cu") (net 3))
 (segment (start 145.55 92.5625) (end 145.55 91.212445) (width 0.2) (layer "F.Cu") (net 3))
 (segment (start 146.35 90.312445) (end 146.4 90.362445) (width 0.2) (layer "F.Cu") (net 3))
 (segment (start 146.4 90.362445) (end 146.5625 90.362445) (width 0.2) (layer "F.Cu") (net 3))
 (segment (start 145.55 91.212445) (end 146.4 90.362445) (width 0.2) (layer "F.Cu") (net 3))
 (segment (start 154 94.375) (end 154.665 95.04) (width 0.2) (layer "F.Cu") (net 7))
 (segment (start 154.665 95.04) (end 160 95.04) (width 0.2) (layer "F.Cu") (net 7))
 (segment (start 147.8375 92.175) (end 149.5 92.175) (width 0.2) (layer "F.Cu") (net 2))
 (segment (start 147.45 92.5625) (end 147.8375 92.175) (width 0.2) (layer "F.Cu") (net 2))
 (segment (start 151.725 93.825) (end 153.05 92.5) (width 0.2) (layer "F.Cu") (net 1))
 (segment (start 149.5 93.825) (end 151 93.825) (width 0.2) (layer "F.Cu") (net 1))
 (segment (start 149.5 93.825) (end 149.5 93.675) (width 0.2) (layer "F.Cu") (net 1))
 (segment (start 151 93.825) (end 151.725 93.825) (width 0.2) (layer "F.Cu") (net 1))
 (segment (start 148 87.362445) (end 148 86.687445) (width 0.2) (layer "F.Cu") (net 9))
 (segment (start 155.299998 83.335) (end 155.600999 83.636001) (width 0.2) (layer "F.Cu") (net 9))
 (segment (start 154.487499 83.335) (end 155.299998 83.335) (width 0.2) (layer "F.Cu") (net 9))
 (segment (start 148 88.862445) (end 148 87.362445) (width 0.2) (layer "F.Cu") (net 9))
 (segment (start 155.600999 84.945968) (end 155.600999 83.636001) (width 0.2) (layer "F.Cu") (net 9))
 (segment (start 154.696967 85.85) (end 148.837445 85.85) (width 0.2) (layer "F.Cu") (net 9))
 (segment (start 155.600999 84.945968) (end 154.696967 85.85) (width 0.2) (layer "F.Cu") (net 9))
 (segment (start 148 86.687445) (end 148.837445 85.85) (width 0.2) (layer "F.Cu") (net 9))
 (segment (start 148.4 84.605) (end 148.026 84.231) (width 0.2) (layer "F.Cu") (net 11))
 (segment (start 149.212499 84.605) (end 148.4 84.605) (width 0.2) (layer "F.Cu") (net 11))
 (segment (start 148.026 81.7681) (end 147.325 81.0671) (width 0.2) (layer "F.Cu") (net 11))
 (segment (start 148.026 84.231) (end 148.026 81.7681) (width 0.2) (layer "F.Cu") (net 11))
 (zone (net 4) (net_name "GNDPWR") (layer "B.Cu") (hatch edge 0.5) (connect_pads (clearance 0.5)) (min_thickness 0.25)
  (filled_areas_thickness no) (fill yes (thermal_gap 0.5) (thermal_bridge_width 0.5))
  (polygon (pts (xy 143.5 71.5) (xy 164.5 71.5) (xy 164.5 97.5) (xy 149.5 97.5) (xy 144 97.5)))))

